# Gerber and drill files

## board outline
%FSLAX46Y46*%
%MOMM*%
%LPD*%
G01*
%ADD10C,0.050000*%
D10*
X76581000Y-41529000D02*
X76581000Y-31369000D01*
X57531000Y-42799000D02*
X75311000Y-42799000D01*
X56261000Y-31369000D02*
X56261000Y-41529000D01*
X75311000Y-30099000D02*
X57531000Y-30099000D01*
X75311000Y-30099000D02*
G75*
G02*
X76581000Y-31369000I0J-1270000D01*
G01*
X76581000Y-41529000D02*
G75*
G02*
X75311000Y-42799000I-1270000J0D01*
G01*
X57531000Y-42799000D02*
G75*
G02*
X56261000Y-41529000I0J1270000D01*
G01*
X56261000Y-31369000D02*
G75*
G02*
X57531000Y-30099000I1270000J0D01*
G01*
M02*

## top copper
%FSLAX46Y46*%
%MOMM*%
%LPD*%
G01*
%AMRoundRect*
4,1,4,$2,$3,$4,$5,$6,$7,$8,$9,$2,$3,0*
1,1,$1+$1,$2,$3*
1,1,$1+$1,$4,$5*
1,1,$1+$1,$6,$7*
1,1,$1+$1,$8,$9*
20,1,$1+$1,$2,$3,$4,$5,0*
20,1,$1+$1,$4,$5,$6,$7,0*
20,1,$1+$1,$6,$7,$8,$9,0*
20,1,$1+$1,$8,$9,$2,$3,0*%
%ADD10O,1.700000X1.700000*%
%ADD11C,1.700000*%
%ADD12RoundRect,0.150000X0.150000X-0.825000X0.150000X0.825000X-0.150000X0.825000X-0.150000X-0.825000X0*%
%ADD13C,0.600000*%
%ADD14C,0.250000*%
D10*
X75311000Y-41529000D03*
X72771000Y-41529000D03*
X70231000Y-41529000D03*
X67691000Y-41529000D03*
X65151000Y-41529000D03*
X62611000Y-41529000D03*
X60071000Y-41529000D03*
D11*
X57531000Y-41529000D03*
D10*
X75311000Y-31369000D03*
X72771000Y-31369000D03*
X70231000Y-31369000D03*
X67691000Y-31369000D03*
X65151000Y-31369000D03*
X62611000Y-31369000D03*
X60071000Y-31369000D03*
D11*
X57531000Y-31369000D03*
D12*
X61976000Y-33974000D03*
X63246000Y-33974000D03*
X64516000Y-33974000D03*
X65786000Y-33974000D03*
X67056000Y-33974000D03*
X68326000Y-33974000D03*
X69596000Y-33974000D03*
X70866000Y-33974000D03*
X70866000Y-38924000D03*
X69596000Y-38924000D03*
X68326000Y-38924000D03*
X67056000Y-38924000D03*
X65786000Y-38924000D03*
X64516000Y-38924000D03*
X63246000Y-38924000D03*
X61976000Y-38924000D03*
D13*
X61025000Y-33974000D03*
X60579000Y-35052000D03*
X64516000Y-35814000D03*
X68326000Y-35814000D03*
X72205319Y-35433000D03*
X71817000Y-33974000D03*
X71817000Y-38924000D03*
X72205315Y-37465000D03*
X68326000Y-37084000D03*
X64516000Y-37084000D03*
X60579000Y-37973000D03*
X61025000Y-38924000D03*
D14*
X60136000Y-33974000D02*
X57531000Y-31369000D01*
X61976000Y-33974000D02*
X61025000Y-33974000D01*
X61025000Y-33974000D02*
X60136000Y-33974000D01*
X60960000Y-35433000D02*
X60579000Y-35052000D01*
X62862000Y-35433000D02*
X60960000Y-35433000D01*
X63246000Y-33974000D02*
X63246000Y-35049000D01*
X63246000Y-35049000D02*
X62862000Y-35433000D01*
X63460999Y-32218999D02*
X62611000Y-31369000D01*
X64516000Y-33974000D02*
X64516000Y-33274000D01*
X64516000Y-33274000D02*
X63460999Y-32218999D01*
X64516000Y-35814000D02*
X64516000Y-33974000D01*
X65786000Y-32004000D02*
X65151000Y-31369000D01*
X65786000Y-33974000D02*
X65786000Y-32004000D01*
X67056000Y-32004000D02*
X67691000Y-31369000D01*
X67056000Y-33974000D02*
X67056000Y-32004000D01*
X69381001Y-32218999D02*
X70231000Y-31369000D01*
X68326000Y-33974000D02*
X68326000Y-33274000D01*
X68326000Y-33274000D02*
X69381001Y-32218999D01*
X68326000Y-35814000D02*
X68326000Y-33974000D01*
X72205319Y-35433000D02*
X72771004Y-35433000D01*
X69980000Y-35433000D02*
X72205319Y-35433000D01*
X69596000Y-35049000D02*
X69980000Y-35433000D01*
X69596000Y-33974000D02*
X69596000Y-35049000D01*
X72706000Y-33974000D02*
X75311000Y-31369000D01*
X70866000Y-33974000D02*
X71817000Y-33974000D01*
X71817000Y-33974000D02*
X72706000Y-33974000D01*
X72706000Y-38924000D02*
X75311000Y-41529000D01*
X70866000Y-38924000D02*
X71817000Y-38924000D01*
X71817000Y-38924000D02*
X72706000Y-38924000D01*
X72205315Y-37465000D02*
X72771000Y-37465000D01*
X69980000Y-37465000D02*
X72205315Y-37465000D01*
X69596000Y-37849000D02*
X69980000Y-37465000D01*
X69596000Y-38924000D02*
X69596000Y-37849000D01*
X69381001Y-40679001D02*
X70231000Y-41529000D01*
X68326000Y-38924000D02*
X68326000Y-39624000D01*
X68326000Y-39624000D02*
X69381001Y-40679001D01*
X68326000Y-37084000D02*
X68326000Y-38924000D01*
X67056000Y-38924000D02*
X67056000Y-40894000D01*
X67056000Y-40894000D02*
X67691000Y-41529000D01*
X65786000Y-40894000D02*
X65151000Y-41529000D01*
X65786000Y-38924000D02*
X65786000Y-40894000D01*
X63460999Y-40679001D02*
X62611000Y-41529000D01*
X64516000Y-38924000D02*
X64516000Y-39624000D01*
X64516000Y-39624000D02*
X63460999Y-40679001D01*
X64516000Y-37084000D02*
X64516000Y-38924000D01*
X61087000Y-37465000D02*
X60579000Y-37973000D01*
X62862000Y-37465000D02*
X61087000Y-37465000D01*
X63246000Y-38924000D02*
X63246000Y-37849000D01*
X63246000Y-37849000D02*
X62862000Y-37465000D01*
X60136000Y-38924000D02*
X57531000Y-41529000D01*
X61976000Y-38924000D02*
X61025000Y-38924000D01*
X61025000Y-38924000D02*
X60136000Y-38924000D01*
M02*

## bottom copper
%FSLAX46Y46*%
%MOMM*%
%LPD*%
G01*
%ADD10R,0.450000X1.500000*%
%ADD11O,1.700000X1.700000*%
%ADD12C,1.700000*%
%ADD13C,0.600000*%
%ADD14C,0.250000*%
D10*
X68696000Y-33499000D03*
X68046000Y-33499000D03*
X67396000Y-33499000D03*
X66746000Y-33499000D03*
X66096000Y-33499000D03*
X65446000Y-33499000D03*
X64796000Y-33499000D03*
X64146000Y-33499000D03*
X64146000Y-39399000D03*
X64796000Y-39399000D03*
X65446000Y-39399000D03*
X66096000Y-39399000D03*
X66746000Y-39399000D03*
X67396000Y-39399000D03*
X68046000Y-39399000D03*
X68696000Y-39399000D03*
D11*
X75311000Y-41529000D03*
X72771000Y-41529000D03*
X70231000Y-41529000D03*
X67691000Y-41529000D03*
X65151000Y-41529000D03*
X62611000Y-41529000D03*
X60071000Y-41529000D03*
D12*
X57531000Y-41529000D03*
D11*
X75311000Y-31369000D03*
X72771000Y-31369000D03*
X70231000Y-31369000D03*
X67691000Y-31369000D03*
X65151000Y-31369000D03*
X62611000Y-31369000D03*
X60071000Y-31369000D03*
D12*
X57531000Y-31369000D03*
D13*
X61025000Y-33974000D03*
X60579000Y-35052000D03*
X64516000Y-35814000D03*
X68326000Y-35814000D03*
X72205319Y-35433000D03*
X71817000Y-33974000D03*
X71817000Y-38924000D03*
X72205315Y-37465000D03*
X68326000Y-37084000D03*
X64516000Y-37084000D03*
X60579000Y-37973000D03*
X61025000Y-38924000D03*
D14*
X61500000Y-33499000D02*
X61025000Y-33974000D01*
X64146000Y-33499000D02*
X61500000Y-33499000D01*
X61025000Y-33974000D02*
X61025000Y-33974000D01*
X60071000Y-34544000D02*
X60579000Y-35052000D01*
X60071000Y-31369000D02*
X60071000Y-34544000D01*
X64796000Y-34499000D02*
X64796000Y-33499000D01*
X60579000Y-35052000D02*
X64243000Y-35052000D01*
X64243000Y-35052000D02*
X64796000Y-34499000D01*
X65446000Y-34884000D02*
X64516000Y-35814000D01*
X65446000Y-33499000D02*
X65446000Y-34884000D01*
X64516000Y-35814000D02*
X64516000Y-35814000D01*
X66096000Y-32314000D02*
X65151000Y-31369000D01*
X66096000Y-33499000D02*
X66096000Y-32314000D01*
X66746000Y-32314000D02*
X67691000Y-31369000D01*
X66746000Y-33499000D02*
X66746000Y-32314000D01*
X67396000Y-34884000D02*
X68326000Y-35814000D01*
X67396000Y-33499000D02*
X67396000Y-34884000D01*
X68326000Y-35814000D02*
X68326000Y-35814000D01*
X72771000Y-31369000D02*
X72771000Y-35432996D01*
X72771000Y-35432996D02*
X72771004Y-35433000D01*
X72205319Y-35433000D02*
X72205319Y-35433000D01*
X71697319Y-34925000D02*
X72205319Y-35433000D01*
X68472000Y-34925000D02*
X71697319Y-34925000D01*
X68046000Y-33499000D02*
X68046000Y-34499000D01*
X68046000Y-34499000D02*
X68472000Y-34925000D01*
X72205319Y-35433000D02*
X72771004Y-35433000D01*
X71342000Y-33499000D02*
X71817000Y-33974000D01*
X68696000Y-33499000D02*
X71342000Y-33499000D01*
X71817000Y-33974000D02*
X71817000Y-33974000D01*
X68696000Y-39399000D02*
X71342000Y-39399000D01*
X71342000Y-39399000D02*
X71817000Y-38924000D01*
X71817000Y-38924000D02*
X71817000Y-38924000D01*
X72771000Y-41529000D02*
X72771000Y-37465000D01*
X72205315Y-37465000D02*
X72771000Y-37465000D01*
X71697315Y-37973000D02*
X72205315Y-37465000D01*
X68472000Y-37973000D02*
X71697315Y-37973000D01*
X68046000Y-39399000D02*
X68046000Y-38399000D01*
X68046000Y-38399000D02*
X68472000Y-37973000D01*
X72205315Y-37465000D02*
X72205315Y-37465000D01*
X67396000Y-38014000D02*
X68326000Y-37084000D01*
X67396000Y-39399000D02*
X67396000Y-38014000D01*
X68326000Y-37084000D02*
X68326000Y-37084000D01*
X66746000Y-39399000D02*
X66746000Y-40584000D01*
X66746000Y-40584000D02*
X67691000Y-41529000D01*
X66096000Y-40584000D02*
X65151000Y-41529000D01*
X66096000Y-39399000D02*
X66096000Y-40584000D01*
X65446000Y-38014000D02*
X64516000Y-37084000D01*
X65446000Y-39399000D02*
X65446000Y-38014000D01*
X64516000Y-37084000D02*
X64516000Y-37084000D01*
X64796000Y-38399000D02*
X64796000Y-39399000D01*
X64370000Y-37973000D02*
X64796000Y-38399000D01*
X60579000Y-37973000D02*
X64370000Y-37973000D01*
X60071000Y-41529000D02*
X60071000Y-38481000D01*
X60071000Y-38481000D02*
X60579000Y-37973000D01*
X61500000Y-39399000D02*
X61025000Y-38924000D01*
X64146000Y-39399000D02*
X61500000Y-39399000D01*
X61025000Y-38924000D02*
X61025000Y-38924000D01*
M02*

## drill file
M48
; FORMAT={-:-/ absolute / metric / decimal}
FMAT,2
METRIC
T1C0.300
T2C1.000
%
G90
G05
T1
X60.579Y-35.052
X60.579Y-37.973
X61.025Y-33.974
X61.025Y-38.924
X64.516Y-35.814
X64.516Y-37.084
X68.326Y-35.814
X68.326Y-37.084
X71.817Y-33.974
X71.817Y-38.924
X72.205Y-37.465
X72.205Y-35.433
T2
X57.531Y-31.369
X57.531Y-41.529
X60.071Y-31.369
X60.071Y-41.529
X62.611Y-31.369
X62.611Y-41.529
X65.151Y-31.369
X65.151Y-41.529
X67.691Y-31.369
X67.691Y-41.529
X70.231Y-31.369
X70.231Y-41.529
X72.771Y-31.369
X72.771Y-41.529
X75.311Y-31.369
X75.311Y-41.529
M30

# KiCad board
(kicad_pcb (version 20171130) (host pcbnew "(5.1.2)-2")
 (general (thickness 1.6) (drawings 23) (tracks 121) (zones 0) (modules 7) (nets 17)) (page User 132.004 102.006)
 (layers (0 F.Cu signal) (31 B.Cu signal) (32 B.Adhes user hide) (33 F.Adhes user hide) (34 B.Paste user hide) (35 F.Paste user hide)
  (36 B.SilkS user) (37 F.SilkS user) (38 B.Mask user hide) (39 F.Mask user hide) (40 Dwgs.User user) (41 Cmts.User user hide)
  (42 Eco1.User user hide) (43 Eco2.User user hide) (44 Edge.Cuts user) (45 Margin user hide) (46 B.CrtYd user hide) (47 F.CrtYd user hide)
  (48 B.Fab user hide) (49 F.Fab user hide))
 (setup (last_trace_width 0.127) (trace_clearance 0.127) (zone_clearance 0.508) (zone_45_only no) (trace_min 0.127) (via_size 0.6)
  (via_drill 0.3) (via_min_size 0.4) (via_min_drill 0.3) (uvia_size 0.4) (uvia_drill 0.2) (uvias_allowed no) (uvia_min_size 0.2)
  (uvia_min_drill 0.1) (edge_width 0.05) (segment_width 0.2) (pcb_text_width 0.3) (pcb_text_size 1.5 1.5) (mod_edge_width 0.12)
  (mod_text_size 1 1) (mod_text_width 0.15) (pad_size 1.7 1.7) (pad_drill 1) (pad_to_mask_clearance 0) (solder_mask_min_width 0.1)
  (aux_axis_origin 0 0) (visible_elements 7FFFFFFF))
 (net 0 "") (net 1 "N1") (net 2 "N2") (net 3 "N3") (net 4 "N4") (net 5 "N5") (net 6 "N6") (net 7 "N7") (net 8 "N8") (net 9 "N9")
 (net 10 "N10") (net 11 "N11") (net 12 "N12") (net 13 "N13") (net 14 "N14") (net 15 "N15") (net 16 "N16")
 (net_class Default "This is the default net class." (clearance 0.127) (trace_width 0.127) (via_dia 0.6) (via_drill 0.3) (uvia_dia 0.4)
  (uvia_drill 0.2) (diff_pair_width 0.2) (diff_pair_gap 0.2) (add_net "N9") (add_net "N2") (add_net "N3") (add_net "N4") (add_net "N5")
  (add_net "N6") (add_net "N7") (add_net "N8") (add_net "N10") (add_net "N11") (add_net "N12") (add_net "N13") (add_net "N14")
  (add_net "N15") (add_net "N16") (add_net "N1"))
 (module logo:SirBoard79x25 (layer F.Cu) (at 66.421 36.449)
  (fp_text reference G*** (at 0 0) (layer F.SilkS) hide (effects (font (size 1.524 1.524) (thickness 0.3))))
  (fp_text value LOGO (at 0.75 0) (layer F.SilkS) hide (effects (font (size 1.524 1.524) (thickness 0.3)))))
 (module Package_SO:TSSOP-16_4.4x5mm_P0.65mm (layer B.Cu) (at 66.421 36.449 90)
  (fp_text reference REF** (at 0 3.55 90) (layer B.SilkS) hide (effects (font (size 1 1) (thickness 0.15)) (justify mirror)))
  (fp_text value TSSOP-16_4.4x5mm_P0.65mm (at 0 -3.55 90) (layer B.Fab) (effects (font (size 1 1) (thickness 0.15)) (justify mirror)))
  (pad 16 smd rect (at 2.95 2.275 90) (size 1.5 0.45) (layers B.Cu B.Paste B.Mask) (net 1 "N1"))
  (pad 15 smd rect (at 2.95 1.625 90) (size 1.5 0.45) (layers B.Cu B.Paste B.Mask) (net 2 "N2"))
  (pad 14 smd rect (at 2.95 0.975 90) (size 1.5 0.45) (layers B.Cu B.Paste B.Mask) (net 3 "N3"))
  (pad 13 smd rect (at 2.95 0.325 90) (size 1.5 0.45) (layers B.Cu B.Paste B.Mask) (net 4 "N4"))
  (pad 12 smd rect (at 2.95 -0.325 90) (size 1.5 0.45) (layers B.Cu B.Paste B.Mask) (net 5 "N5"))
  (pad 11 smd rect (at 2.95 -0.975 90) (size 1.5 0.45) (layers B.Cu B.Paste B.Mask) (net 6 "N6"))
  (pad 10 smd rect (at 2.95 -1.625 90) (size 1.5 0.45) (layers B.Cu B.Paste B.Mask) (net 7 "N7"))
  (pad 9 smd rect (at 2.95 -2.275 90) (size 1.5 0.45) (layers B.Cu B.Paste B.Mask) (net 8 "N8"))
  (pad 8 smd rect (at -2.95 -2.275 90) (size 1.5 0.45) (layers B.Cu B.Paste B.Mask) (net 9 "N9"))
  (pad 7 smd rect (at -2.95 -1.625 90) (size 1.5 0.45) (layers B.Cu B.Paste B.Mask) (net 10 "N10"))
  (pad 6 smd rect (at -2.95 -0.975 90) (size 1.5 0.45) (layers B.Cu B.Paste B.Mask) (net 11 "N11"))
  (pad 5 smd rect (at -2.95 -0.325 90) (size 1.5 0.45) (layers B.Cu B.Paste B.Mask) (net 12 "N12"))
  (pad 4 smd rect (at -2.95 0.325 90) (size 1.5 0.45) (layers B.Cu B.Paste B.Mask) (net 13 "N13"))
  (pad 3 smd rect (at -2.95 0.975 90) (size 1.5 0.45) (layers B.Cu B.Paste B.Mask) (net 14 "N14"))
  (pad 2 smd rect (at -2.95 1.625 90) (size 1.5 0.45) (layers B.Cu B.Paste B.Mask) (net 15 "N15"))
  (pad 1 smd rect (at -2.95 2.275 90) (size 1.5 0.45) (layers B.Cu B.Paste B.Mask) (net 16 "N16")))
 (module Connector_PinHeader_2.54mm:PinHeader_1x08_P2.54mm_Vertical (layer F.Cu) (at 57.531 41.529 90)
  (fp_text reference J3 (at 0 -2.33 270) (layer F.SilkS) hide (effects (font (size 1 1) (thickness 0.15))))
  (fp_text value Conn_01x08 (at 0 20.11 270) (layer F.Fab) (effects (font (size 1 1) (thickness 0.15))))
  (pad 8 thru_hole oval (at 0 17.78 90) (size 1.7 1.7) (drill 1) (layers *.Cu *.Mask) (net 16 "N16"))
  (pad 7 thru_hole oval (at 0 15.24 90) (size 1.7 1.7) (drill 1) (layers *.Cu *.Mask) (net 15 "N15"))
  (pad 6 thru_hole oval (at 0 12.7 90) (size 1.7 1.7) (drill 1) (layers *.Cu *.Mask) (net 14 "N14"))
  (pad 5 thru_hole oval (at 0 10.16 90) (size 1.7 1.7) (drill 1) (layers *.Cu *.Mask) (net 13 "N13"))
  (pad 4 thru_hole oval (at 0 7.62 90) (size 1.7 1.7) (drill 1) (layers *.Cu *.Mask) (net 12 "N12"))
  (pad 3 thru_hole oval (at 0 5.08 90) (size 1.7 1.7) (drill 1) (layers *.Cu *.Mask) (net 11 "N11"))
  (pad 2 thru_hole oval (at 0 2.54 90) (size 1.7 1.7) (drill 1) (layers *.Cu *.Mask) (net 10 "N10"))
  (pad 1 thru_hole circle (at 0 0 90) (size 1.7 1.7) (drill 1) (layers *.Cu *.Mask) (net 9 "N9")))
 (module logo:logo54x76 (layer F.Cu) (at 58.801 36.449)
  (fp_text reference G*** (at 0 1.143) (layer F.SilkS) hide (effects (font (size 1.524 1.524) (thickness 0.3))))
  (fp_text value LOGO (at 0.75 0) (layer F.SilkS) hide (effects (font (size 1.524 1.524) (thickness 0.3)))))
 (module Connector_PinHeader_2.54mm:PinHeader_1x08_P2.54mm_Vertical (layer F.Cu) (at 57.531 31.369 90)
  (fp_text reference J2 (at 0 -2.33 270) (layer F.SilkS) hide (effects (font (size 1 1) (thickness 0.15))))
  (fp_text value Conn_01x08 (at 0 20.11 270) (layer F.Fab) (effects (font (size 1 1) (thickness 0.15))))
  (pad 8 thru_hole oval (at 0 17.78 90) (size 1.7 1.7) (drill 1) (layers *.Cu *.Mask) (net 1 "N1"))
  (pad 7 thru_hole oval (at 0 15.24 90) (size 1.7 1.7) (drill 1) (layers *.Cu *.Mask) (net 2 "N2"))
  (pad 6 thru_hole oval (at 0 12.7 90) (size 1.7 1.7) (drill 1) (layers *.Cu *.Mask) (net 3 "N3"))
  (pad 5 thru_hole oval (at 0 10.16 90) (size 1.7 1.7) (drill 1) (layers *.Cu *.Mask) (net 4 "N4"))
  (pad 4 thru_hole oval (at 0 7.62 90) (size 1.7 1.7) (drill 1) (layers *.Cu *.Mask) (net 5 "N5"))
  (pad 3 thru_hole oval (at 0 5.08 90) (size 1.7 1.7) (drill 1) (layers *.Cu *.Mask) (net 6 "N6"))
  (pad 2 thru_hole oval (at 0 2.54 90) (size 1.7 1.7) (drill 1) (layers *.Cu *.Mask) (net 7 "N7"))
  (pad 1 thru_hole circle (at 0 0 90) (size 1.7 1.7) (drill 1) (layers *.Cu *.Mask) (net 8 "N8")))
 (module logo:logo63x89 (layer B.Cu) (at 72.771 36.449 180)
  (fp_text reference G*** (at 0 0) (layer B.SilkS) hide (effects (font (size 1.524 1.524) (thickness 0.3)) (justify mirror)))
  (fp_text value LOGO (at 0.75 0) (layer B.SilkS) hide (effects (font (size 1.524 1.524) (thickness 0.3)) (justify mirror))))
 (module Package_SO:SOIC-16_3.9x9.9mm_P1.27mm (layer F.Cu) (at 66.421 36.449 90)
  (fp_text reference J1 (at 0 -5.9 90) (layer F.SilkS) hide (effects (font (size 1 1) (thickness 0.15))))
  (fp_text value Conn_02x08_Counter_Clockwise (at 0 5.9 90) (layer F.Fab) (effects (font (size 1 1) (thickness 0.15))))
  (pad 16 smd roundrect (at 2.475 -4.445 90) (size 1.95 0.6) (layers F.Cu F.Paste F.Mask) (roundrect_rratio 0.25) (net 8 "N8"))
  (pad 15 smd roundrect (at 2.475 -3.175 90) (size 1.95 0.6) (layers F.Cu F.Paste F.Mask) (roundrect_rratio 0.25) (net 7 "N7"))
  (pad 14 smd roundrect (at 2.475 -1.905 90) (size 1.95 0.6) (layers F.Cu F.Paste F.Mask) (roundrect_rratio 0.25) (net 6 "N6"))
  (pad 13 smd roundrect (at 2.475 -0.635 90) (size 1.95 0.6) (layers F.Cu F.Paste F.Mask) (roundrect_rratio 0.25) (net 5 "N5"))
  (pad 12 smd roundrect (at 2.475 0.635 90) (size 1.95 0.6) (layers F.Cu F.Paste F.Mask) (roundrect_rratio 0.25) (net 4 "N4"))
  (pad 11 smd roundrect (at 2.475 1.905 90) (size 1.95 0.6) (layers F.Cu F.Paste F.Mask) (roundrect_rratio 0.25) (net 3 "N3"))
  (pad 10 smd roundrect (at 2.475 3.175 90) (size 1.95 0.6) (layers F.Cu F.Paste F.Mask) (roundrect_rratio 0.25) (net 2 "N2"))
  (pad 9 smd roundrect (at 2.475 4.445 90) (size 1.95 0.6) (layers F.Cu F.Paste F.Mask) (roundrect_rratio 0.25) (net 1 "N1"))
  (pad 8 smd roundrect (at -2.475 4.445 90) (size 1.95 0.6) (layers F.Cu F.Paste F.Mask) (roundrect_rratio 0.25) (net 16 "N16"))
  (pad 7 smd roundrect (at -2.475 3.175 90) (size 1.95 0.6) (layers F.Cu F.Paste F.Mask) (roundrect_rratio 0.25) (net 15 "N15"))
  (pad 6 smd roundrect (at -2.475 1.905 90) (size 1.95 0.6) (layers F.Cu F.Paste F.Mask) (roundrect_rratio 0.25) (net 14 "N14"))
  (pad 5 smd roundrect (at -2.475 0.635 90) (size 1.95 0.6) (layers F.Cu F.Paste F.Mask) (roundrect_rratio 0.25) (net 13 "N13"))
  (pad 4 smd roundrect (at -2.475 -0.635 90) (size 1.95 0.6) (layers F.Cu F.Paste F.Mask) (roundrect_rratio 0.25) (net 12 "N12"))
  (pad 3 smd roundrect (at -2.475 -1.905 90) (size 1.95 0.6) (layers F.Cu F.Paste F.Mask) (roundrect_rratio 0.25) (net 11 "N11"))
  (pad 2 smd roundrect (at -2.475 -3.175 90) (size 1.95 0.6) (layers F.Cu F.Paste F.Mask) (roundrect_rratio 0.25) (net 10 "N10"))
  (pad 1 smd roundrect (at -2.475 -4.445 90) (size 1.95 0.6) (layers F.Cu F.Paste F.Mask) (roundrect_rratio 0.25) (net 9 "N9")))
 (gr_line (start 76.581 41.529) (end 76.581 31.369) (layer Edge.Cuts) (width 0.05))
 (gr_line (start 57.531 42.799) (end 75.311 42.799) (layer Edge.Cuts) (width 0.05))
 (gr_line (start 56.261 31.369) (end 56.261 41.529) (layer Edge.Cuts) (width 0.05))
 (gr_line (start 75.311 30.099) (end 57.531 30.099) (layer Edge.Cuts) (width 0.05))
 (gr_arc (start 75.311 31.369) (end 76.581 31.369) (angle -90) (layer Edge.Cuts) (width 0.05))
 (gr_arc (start 75.311 41.529) (end 75.311 42.799) (angle -90) (layer Edge.Cuts) (width 0.05))
 (gr_arc (start 57.531 41.529) (end 56.261 41.529) (angle -90) (layer Edge.Cuts) (width 0.05))
 (gr_arc (start 57.531 31.369) (end 57.531 30.099) (angle -90) (layer Edge.Cuts) (width 0.05))
 (segment (start 60.136 33.974) (end 57.531 31.369) (width 0.25) (layer F.Cu) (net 8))
 (segment (start 61.5 33.499) (end 61.025 33.974) (width 0.25) (layer B.Cu) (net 8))
 (segment (start 64.146 33.499) (end 61.5 33.499) (width 0.25) (layer B.Cu) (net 8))
 (segment (start 61.976 33.974) (end 61.025 33.974) (width 0.25) (layer F.Cu) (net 8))
 (segment (start 61.025 33.974) (end 60.136 33.974) (width 0.25) (layer F.Cu) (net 8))
 (segment (start 61.025 33.974) (end 61.025 33.974) (width 0.25) (layer B.Cu) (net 8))
 (via (at 61.025 33.974) (size 0.6) (drill 0.3) (layers F.Cu B.Cu) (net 8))
 (via (at 60.579 35.052) (size 0.6) (drill 0.3) (layers F.Cu B.Cu) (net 7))
 (segment (start 60.071 34.544) (end 60.579 35.052) (width 0.25) (layer B.Cu) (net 7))
 (segment (start 60.071 31.369) (end 60.071 34.544) (width 0.25) (layer B.Cu) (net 7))
 (segment (start 64.796 34.499) (end 64.796 33.499) (width 0.25) (layer B.Cu) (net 7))
 (segment (start 60.579 35.052) (end 64.243 35.052) (width 0.25) (layer B.Cu) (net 7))
 (segment (start 64.243 35.052) (end 64.796 34.499) (width 0.25) (layer B.Cu) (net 7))
 (segment (start 60.96 35.433) (end 60.579 35.052) (width 0.25) (layer F.Cu) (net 7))
 (segment (start 62.862 35.433) (end 60.96 35.433) (width 0.25) (layer F.Cu) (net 7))
 (segment (start 63.246 33.974) (end 63.246 35.049) (width 0.25) (layer F.Cu) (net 7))
 (segment (start 63.246 35.049) (end 62.862 35.433) (width 0.25) (layer F.Cu) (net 7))
 (segment (start 63.460999 32.218999) (end 62.611 31.369) (width 0.25) (layer F.Cu) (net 6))
 (segment (start 64.516 33.974) (end 64.516 33.274) (width 0.25) (layer F.Cu) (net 6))
 (segment (start 64.516 33.274) (end 63.460999 32.218999) (width 0.25) (layer F.Cu) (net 6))
 (segment (start 65.446 34.884) (end 64.516 35.814) (width 0.25) (layer B.Cu) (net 6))
 (segment (start 65.446 33.499) (end 65.446 34.884) (width 0.25) (layer B.Cu) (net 6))
 (segment (start 64.516 35.814) (end 64.516 33.974) (width 0.25) (layer F.Cu) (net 6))
 (segment (start 64.516 35.814) (end 64.516 35.814) (width 0.25) (layer B.Cu) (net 6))
 (via (at 64.516 35.814) (size 0.6) (drill 0.3) (layers F.Cu B.Cu) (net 6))
 (segment (start 65.786 32.004) (end 65.151 31.369) (width 0.25) (layer F.Cu) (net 5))
 (segment (start 65.786 33.974) (end 65.786 32.004) (width 0.25) (layer F.Cu) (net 5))
 (segment (start 66.096 32.314) (end 65.151 31.369) (width 0.25) (layer B.Cu) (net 5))
 (segment (start 66.096 33.499) (end 66.096 32.314) (width 0.25) (layer B.Cu) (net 5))
 (segment (start 67.056 32.004) (end 67.691 31.369) (width 0.25) (layer F.Cu) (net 4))
 (segment (start 67.056 33.974) (end 67.056 32.004) (width 0.25) (layer F.Cu) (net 4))
 (segment (start 66.746 32.314) (end 67.691 31.369) (width 0.25) (layer B.Cu) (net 4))
 (segment (start 66.746 33.499) (end 66.746 32.314) (width 0.25) (layer B.Cu) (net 4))
 (segment (start 69.381001 32.218999) (end 70.231 31.369) (width 0.25) (layer F.Cu) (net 3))
 (segment (start 68.326 33.974) (end 68.326 33.274) (width 0.25) (layer F.Cu) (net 3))
 (segment (start 68.326 33.274) (end 69.381001 32.218999) (width 0.25) (layer F.Cu) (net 3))
 (segment (start 67.396 34.884) (end 68.326 35.814) (width 0.25) (layer B.Cu) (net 3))
 (segment (start 67.396 33.499) (end 67.396 34.884) (width 0.25) (layer B.Cu) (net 3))
 (segment (start 68.326 35.814) (end 68.326 33.974) (width 0.25) (layer F.Cu) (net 3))
 (segment (start 68.326 35.814) (end 68.326 35.814) (width 0.25) (layer B.Cu) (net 3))
 (via (at 68.326 35.814) (size 0.6) (drill 0.3) (layers F.Cu B.Cu) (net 3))
 (segment (start 72.205319 35.433) (end 72.771004 35.433) (width 0.25) (layer F.Cu) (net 2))
 (segment (start 69.98 35.433) (end 72.205319 35.433) (width 0.25) (layer F.Cu) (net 2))
 (segment (start 69.596 35.049) (end 69.98 35.433) (width 0.25) (layer F.Cu) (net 2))
 (segment (start 69.596 33.974) (end 69.596 35.049) (width 0.25) (layer F.Cu) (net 2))
 (segment (start 72.771 31.369) (end 72.771 35.432996) (width 0.25) (layer B.Cu) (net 2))
 (segment (start 72.771 35.432996) (end 72.771004 35.433) (width 0.25) (layer B.Cu) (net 2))
 (segment (start 72.205319 35.433) (end 72.205319 35.433) (width 0.25) (layer B.Cu) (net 2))
 (segment (start 71.697319 34.925) (end 72.205319 35.433) (width 0.25) (layer B.Cu) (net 2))
 (segment (start 68.472 34.925) (end 71.697319 34.925) (width 0.25) (layer B.Cu) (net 2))
 (segment (start 68.046 33.499) (end 68.046 34.499) (width 0.25) (layer B.Cu) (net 2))
 (segment (start 68.046 34.499) (end 68.472 34.925) (width 0.25) (layer B.Cu) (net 2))
 (segment (start 72.205319 35.433) (end 72.771004 35.433) (width 0.25) (layer B.Cu) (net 2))
 (via (at 72.205319 35.433) (size 0.6) (drill 0.3) (layers F.Cu B.Cu) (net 2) (status 1000000))
 (segment (start 72.706 33.974) (end 75.311 31.369) (width 0.25) (layer F.Cu) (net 1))
 (segment (start 71.342 33.499) (end 71.817 33.974) (width 0.25) (layer B.Cu) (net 1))
 (segment (start 68.696 33.499) (end 71.342 33.499) (width 0.25) (layer B.Cu) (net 1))
 (segment (start 70.866 33.974) (end 71.817 33.974) (width 0.25) (layer F.Cu) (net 1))
 (segment (start 71.817 33.974) (end 72.706 33.974) (width 0.25) (layer F.Cu) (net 1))
 (segment (start 71.817 33.974) (end 71.817 33.974) (width 0.25) (layer B.Cu) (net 1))
 (via (at 71.817 33.974) (size 0.6) (drill 0.3) (layers F.Cu B.Cu) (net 1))
 (segment (start 72.706 38.924) (end 75.311 41.529) (width 0.25) (layer F.Cu) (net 16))
 (segment (start 68.696 39.399) (end 71.342 39.399) (width 0.25) (layer B.Cu) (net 16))
 (segment (start 71.342 39.399) (end 71.817 38.924) (width 0.25) (layer B.Cu) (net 16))
 (segment (start 70.866 38.924) (end 71.817 38.924) (width 0.25) (layer F.Cu) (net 16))
 (segment (start 71.817 38.924) (end 72.706 38.924) (width 0.25) (layer F.Cu) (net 16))
 (segment (start 71.817 38.924) (end 71.817 38.924) (width 0.25) (layer B.Cu) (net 16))
 (via (at 71.817 38.924) (size 0.6) (drill 0.3) (layers F.Cu B.Cu) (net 16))
 (segment (start 72.771 41.529) (end 72.771 37.465) (width 0.25) (layer B.Cu) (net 15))
 (segment (start 72.205315 37.465) (end 72.771 37.465) (width 0.25) (layer F.Cu) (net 15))
 (segment (start 69.98 37.465) (end 72.205315 37.465) (width 0.25) (layer F.Cu) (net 15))
 (segment (start 69.596 37.849) (end 69.98 37.465) (width 0.25) (layer F.Cu) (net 15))
 (segment (start 69.596 38.924) (end 69.596 37.849) (width 0.25) (layer F.Cu) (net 15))
 (segment (start 72.205315 37.465) (end 72.771 37.465) (width 0.25) (layer B.Cu) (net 15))
 (segment (start 71.697315 37.973) (end 72.205315 37.465) (width 0.25) (layer B.Cu) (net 15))
 (segment (start 68.472 37.973) (end 71.697315 37.973) (width 0.25) (layer B.Cu) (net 15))
 (segment (start 68.046 39.399) (end 68.046 38.399) (width 0.25) (layer B.Cu) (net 15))
 (segment (start 68.046 38.399) (end 68.472 37.973) (width 0.25) (layer B.Cu) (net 15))
 (segment (start 72.205315 37.465) (end 72.205315 37.465) (width 0.25) (layer B.Cu) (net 15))
 (via (at 72.205315 37.465) (size 0.6) (drill 0.3) (layers F.Cu B.Cu) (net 15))
 (segment (start 69.381001 40.679001) (end 70.231 41.529) (width 0.25) (layer F.Cu) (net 14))
 (segment (start 68.326 38.924) (end 68.326 39.624) (width 0.25) (layer F.Cu) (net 14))
 (segment (start 68.326 39.624) (end 69.381001 40.679001) (width 0.25) (layer F.Cu) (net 14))
 (segment (start 67.396 38.014) (end 68.326 37.084) (width 0.25) (layer B.Cu) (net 14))
 (segment (start 67.396 39.399) (end 67.396 38.014) (width 0.25) (layer B.Cu) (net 14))
 (segment (start 68.326 37.084) (end 68.326 38.924) (width 0.25) (layer F.Cu) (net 14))
 (segment (start 68.326 37.084) (end 68.326 37.084) (width 0.25) (layer B.Cu) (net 14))
 (via (at 68.326 37.084) (size 0.6) (drill 0.3) (layers F.Cu B.Cu) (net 14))
 (segment (start 66.746 39.399) (end 66.746 40.584) (width 0.25) (layer B.Cu) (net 13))
 (segment (start 66.746 40.584) (end 67.691 41.529) (width 0.25) (layer B.Cu) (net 13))
 (segment (start 67.056 38.924) (end 67.056 40.894) (width 0.25) (layer F.Cu) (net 13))
 (segment (start 67.056 40.894) (end 67.691 41.529) (width 0.25) (layer F.Cu) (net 13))
 (segment (start 65.786 40.894) (end 65.151 41.529) (width 0.25) (layer F.Cu) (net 12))
 (segment (start 65.786 38.924) (end 65.786 40.894) (width 0.25) (layer F.Cu) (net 12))
 (segment (start 66.096 40.584) (end 65.151 41.529) (width 0.25) (layer B.Cu) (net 12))
 (segment (start 66.096 39.399) (end 66.096 40.584) (width 0.25) (layer B.Cu) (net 12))
 (segment (start 63.460999 40.679001) (end 62.611 41.529) (width 0.25) (layer F.Cu) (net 11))
 (segment (start 64.516 38.924) (end 64.516 39.624) (width 0.25) (layer F.Cu) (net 11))
 (segment (start 64.516 39.624) (end 63.460999 40.679001) (width 0.25) (layer F.Cu) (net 11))
 (segment (start 64.516 37.084) (end 64.516 38.924) (width 0.25) (layer F.Cu) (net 11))
 (segment (start 65.446 38.014) (end 64.516 37.084) (width 0.25) (layer B.Cu) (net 11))
 (segment (start 65.446 39.399) (end 65.446 38.014) (width 0.25) (layer B.Cu) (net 11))
 (segment (start 64.516 37.084) (end 64.516 37.084) (width 0.25) (layer B.Cu) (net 11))
 (via (at 64.516 37.084) (size 0.6) (drill 0.3) (layers F.Cu B.Cu) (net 11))
 (via (at 60.579 37.973) (size 0.6) (drill 0.3) (layers F.Cu B.Cu) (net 10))
 (segment (start 64.796 38.399) (end 64.796 39.399) (width 0.25) (layer B.Cu) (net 10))
 (segment (start 64.37 37.973) (end 64.796 38.399) (width 0.25) (layer B.Cu) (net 10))
 (segment (start 60.579 37.973) (end 64.37 37.973) (width 0.25) (layer B.Cu) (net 10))
 (segment (start 60.071 41.529) (end 60.071 38.481) (width 0.25) (layer B.Cu) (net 10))
 (segment (start 60.071 38.481) (end 60.579 37.973) (width 0.25) (layer B.Cu) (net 10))
 (segment (start 61.087 37.465) (end 60.579 37.973) (width 0.25) (layer F.Cu) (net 10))
 (segment (start 62.862 37.465) (end 61.087 37.465) (width 0.25) (layer F.Cu) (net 10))
 (segment (start 63.246 38.924) (end 63.246 37.849) (width 0.25) (layer F.Cu) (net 10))
 (segment (start 63.246 37.849) (end 62.862 37.465) (width 0.25) (layer F.Cu) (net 10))
 (segment (start 60.136 38.924) (end 57.531 41.529) (width 0.25) (layer F.Cu) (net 9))
 (segment (start 61.5 39.399) (end 61.025 38.924) (width 0.25) (layer B.Cu) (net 9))
 (segment (start 61.976 38.924) (end 61.025 38.924) (width 0.25) (layer F.Cu) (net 9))
 (segment (start 61.025 38.924) (end 60.136 38.924) (width 0.25) (layer F.Cu) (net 9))
 (segment (start 64.146 39.399) (end 61.5 39.399) (width 0.25) (layer B.Cu) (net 9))
 (segment (start 61.025 38.924) (end 61.025 38.924) (width 0.25) (layer B.Cu) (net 9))
 (via (at 61.025 38.924) (size 0.6) (drill 0.3) (layers F.Cu B.Cu) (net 9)))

